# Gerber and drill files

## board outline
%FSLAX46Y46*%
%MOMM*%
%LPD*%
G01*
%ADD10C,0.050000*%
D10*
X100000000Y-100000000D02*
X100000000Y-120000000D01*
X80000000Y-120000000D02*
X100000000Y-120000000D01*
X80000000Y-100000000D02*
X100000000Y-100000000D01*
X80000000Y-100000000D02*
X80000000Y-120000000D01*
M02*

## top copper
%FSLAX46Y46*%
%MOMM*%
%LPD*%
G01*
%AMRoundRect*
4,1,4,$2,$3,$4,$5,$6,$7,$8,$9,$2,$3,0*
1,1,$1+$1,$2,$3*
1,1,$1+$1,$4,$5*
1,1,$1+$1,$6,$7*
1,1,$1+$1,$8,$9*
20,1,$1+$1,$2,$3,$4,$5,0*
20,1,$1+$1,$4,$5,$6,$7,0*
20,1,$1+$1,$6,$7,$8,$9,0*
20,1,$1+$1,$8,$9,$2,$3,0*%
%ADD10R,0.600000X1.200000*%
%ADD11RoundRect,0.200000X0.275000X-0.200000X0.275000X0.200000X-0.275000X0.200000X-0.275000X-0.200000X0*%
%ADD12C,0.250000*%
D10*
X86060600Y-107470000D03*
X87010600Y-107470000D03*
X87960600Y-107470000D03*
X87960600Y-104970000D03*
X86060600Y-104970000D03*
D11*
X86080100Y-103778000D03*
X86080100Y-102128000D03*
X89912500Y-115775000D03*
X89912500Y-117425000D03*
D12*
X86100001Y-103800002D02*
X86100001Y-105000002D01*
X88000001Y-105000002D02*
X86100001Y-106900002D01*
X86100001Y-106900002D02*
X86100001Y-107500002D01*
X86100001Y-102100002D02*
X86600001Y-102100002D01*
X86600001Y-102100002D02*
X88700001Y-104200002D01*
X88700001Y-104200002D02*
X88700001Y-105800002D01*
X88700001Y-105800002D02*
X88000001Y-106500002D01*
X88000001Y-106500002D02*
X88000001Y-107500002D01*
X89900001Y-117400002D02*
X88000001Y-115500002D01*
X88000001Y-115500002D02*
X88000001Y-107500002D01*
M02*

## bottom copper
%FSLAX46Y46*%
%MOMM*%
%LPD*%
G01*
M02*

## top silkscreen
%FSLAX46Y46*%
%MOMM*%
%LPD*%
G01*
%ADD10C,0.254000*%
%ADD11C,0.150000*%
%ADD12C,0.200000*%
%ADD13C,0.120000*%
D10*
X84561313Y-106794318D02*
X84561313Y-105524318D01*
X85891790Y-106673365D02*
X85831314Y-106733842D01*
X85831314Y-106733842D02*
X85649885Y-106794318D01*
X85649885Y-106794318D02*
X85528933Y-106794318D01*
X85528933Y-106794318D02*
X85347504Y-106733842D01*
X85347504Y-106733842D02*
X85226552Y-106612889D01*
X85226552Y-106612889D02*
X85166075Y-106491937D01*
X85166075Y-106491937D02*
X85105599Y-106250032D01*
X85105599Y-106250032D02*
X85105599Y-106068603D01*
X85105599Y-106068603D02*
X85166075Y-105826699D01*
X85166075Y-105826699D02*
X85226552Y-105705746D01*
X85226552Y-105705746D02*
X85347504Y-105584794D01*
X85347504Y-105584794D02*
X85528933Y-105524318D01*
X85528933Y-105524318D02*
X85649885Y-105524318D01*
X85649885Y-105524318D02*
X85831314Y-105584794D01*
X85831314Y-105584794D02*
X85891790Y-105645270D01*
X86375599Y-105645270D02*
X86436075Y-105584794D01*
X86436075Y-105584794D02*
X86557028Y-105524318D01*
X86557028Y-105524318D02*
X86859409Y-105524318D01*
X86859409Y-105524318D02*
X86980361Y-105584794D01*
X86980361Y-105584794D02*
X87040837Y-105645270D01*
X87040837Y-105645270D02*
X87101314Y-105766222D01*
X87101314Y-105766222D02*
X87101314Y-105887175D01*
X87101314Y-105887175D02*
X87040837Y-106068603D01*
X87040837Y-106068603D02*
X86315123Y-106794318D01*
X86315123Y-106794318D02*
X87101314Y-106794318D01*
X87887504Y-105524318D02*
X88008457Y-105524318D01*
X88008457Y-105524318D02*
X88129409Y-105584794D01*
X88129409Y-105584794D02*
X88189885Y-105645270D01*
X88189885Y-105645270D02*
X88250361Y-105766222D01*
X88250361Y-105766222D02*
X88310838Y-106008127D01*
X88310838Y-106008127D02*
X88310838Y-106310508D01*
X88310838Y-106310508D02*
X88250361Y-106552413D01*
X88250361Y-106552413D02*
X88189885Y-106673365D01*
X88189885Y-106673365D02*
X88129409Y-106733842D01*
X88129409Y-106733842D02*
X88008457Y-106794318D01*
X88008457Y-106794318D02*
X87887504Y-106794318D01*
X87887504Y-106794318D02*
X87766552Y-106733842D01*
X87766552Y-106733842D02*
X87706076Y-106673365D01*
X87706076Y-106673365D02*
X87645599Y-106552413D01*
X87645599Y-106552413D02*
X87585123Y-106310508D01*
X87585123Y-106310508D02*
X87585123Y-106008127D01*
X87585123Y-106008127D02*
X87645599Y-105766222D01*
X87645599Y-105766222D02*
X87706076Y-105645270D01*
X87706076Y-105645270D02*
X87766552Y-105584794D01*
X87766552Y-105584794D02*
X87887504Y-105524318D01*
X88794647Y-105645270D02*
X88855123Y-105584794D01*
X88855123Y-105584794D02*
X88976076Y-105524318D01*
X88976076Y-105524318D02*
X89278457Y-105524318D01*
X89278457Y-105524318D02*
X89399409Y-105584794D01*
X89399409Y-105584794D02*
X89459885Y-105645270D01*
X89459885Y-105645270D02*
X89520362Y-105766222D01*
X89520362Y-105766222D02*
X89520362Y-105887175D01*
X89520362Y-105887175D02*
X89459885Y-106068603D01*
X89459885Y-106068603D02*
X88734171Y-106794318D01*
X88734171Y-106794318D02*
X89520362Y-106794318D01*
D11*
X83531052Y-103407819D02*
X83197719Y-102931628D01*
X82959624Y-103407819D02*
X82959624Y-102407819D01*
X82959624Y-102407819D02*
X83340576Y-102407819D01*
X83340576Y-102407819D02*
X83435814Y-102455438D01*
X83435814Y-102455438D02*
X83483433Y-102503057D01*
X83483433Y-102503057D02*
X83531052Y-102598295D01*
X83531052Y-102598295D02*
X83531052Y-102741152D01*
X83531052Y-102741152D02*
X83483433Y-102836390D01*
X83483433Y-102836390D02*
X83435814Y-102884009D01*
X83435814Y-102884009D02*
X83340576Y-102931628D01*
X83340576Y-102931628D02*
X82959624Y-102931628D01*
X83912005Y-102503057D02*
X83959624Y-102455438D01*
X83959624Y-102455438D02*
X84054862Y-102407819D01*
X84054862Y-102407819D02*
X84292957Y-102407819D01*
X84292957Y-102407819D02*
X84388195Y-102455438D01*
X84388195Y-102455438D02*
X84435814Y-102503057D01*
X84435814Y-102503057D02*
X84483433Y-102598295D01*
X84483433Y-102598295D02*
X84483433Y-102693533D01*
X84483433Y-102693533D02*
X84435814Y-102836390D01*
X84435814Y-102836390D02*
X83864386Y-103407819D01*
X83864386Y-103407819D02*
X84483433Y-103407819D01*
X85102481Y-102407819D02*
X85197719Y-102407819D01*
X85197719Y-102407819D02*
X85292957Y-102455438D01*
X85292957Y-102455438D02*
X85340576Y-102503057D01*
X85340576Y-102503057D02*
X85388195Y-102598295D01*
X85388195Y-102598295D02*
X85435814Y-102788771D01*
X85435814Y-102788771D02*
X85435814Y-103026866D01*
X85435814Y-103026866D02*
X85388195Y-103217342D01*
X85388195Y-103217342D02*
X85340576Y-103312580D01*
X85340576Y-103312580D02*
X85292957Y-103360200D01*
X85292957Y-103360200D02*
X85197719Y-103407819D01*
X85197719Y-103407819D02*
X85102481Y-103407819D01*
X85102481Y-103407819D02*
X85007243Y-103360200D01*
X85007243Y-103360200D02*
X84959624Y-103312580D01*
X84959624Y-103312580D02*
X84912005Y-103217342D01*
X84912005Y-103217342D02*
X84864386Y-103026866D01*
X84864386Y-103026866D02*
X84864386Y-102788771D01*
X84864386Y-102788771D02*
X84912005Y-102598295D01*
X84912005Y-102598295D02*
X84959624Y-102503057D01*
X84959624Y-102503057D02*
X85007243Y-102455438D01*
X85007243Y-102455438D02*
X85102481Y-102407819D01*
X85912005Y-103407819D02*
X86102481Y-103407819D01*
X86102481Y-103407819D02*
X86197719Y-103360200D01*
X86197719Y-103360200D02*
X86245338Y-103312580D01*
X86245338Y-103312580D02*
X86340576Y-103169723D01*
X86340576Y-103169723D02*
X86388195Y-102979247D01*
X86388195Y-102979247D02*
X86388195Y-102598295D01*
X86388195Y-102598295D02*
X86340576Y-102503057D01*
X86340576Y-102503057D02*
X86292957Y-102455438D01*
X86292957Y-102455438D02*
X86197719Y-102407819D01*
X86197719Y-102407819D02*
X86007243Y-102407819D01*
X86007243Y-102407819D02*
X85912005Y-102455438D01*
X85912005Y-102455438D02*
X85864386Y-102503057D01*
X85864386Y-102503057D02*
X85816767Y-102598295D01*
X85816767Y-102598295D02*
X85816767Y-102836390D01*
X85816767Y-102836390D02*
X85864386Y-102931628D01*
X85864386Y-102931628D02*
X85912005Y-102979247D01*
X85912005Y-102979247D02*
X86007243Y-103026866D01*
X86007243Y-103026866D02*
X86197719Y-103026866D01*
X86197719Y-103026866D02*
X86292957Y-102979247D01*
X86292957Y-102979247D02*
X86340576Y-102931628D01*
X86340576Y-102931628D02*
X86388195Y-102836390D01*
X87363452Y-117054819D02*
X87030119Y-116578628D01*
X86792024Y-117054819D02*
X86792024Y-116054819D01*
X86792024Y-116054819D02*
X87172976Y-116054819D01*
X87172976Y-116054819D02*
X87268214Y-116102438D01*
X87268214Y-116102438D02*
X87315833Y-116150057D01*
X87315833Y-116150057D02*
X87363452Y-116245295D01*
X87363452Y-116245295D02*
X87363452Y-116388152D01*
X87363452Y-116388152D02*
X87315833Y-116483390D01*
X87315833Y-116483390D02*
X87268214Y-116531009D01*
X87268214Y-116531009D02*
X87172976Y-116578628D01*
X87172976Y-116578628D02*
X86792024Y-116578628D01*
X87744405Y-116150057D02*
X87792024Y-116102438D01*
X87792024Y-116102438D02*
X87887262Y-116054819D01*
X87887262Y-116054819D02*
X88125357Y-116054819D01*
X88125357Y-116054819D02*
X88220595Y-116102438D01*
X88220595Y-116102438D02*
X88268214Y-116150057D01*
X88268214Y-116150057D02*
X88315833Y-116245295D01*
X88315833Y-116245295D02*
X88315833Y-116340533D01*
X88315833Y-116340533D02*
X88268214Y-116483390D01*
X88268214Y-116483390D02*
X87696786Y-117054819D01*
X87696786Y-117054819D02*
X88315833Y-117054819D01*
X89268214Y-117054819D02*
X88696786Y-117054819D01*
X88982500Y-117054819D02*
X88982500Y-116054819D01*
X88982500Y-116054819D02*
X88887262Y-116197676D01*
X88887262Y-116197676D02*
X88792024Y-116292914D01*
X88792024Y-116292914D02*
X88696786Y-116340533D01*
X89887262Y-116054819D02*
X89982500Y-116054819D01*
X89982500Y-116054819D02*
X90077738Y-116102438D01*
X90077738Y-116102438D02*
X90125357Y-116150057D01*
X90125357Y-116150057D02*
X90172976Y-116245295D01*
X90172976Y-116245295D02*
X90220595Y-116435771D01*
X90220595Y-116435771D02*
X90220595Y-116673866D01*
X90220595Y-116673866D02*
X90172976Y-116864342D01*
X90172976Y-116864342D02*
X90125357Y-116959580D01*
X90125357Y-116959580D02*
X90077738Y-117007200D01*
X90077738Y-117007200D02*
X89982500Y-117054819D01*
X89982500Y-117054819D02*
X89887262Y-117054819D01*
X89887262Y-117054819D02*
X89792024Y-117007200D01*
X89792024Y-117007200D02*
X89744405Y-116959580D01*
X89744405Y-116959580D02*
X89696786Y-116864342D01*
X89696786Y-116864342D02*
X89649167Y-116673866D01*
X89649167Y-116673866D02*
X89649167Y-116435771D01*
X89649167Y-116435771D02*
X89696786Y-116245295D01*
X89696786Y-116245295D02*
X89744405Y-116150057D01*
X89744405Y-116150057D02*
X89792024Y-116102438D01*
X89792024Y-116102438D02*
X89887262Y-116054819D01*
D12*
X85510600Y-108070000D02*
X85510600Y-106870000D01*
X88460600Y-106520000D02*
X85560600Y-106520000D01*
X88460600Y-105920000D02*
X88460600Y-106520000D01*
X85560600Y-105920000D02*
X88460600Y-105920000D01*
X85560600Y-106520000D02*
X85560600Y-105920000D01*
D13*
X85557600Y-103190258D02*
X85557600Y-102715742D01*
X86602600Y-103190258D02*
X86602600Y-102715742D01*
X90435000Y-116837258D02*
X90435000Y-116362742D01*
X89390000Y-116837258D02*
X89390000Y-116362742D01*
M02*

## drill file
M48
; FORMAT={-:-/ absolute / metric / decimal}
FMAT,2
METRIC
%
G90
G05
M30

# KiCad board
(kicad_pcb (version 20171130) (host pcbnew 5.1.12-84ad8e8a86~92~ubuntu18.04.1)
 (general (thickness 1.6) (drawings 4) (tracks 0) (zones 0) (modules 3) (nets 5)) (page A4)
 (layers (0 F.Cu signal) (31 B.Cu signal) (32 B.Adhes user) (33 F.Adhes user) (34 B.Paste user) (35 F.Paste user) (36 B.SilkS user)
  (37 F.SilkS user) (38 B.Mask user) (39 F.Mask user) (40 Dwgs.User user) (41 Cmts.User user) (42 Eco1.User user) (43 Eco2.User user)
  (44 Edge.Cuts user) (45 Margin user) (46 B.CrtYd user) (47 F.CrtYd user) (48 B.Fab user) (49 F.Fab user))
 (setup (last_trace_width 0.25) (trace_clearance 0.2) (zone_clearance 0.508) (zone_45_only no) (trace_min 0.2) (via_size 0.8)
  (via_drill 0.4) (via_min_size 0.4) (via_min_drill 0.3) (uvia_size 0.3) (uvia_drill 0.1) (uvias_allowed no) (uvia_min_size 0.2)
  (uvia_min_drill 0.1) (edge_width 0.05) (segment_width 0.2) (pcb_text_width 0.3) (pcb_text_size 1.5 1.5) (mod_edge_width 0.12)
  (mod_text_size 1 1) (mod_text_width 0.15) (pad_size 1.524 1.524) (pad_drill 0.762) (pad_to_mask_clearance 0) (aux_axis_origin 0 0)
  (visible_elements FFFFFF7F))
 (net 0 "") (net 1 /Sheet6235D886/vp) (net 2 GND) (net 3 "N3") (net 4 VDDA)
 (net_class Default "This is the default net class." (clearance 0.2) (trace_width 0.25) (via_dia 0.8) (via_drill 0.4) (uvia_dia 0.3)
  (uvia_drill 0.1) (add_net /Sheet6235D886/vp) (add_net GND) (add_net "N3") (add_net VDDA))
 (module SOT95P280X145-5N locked (layer F.Cu) (at 87.010600 106.220000 90.000000)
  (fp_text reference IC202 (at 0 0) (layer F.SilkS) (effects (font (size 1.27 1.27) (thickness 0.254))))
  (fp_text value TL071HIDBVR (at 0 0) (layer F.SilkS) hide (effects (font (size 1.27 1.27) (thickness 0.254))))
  (fp_line (start -1.85 -1.5) (end -0.65 -1.5) (layer F.SilkS) (width 0.2))
  (fp_line (start -0.3 1.45) (end -0.3 -1.45) (layer F.SilkS) (width 0.2))
  (fp_line (start 0.3 1.45) (end -0.3 1.45) (layer F.SilkS) (width 0.2))
  (fp_line (start 0.3 -1.45) (end 0.3 1.45) (layer F.SilkS) (width 0.2))
  (fp_line (start -0.3 -1.45) (end 0.3 -1.45) (layer F.SilkS) (width 0.2))
  (pad 1 smd rect (at -1.25 -0.95 180.000000) (size 0.6 1.2) (layers F.Cu F.Mask F.Paste) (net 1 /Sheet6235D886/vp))
  (pad 2 smd rect (at -1.25 0 180.000000) (size 0.6 1.2) (layers F.Cu F.Mask F.Paste) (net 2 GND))
  (pad 3 smd rect (at -1.25 0.95 180.000000) (size 0.6 1.2) (layers F.Cu F.Mask F.Paste) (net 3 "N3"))
  (pad 4 smd rect (at 1.25 0.95 180.000000) (size 0.6 1.2) (layers F.Cu F.Mask F.Paste) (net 1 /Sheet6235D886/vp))
  (pad 5 smd rect (at 1.25 -0.95 180.000000) (size 0.6 1.2) (layers F.Cu F.Mask F.Paste) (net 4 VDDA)))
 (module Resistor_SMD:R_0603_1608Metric (layer F.Cu) (at 86.080100 102.953000 90.000000)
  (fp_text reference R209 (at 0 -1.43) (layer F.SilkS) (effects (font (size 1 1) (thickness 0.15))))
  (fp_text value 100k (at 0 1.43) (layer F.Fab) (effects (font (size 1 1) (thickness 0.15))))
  (fp_line (start -0.237258 -0.5225) (end 0.237258 -0.5225) (layer F.SilkS) (width 0.12))
  (fp_line (start -0.237258 0.5225) (end 0.237258 0.5225) (layer F.SilkS) (width 0.12))
  (pad 1 smd roundrect (at -0.825 0 90.000000) (size 0.8 0.95) (layers F.Cu F.Mask F.Paste) (roundrect_rratio 0.25) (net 4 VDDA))
  (pad 2 smd roundrect (at 0.825 0 90.000000) (size 0.8 0.95) (layers F.Cu F.Mask F.Paste) (roundrect_rratio 0.25) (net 3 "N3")))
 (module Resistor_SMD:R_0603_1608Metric (layer F.Cu) (at 89.912500 116.600000 90.000000)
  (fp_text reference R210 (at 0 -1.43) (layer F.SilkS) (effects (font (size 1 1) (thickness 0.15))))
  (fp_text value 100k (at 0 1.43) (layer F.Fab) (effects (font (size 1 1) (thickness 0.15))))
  (fp_line (start -0.237258 0.5225) (end 0.237258 0.5225) (layer F.SilkS) (width 0.12))
  (fp_line (start -0.237258 -0.5225) (end 0.237258 -0.5225) (layer F.SilkS) (width 0.12))
  (pad 2 smd roundrect (at 0.825 0 90.000000) (size 0.8 0.95) (layers F.Cu F.Mask F.Paste) (roundrect_rratio 0.25) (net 2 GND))
  (pad 1 smd roundrect (at -0.825 0 90.000000) (size 0.8 0.95) (layers F.Cu F.Mask F.Paste) (roundrect_rratio 0.25) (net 3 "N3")))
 (gr_line (start 100 100) (end 100 120) (layer Edge.Cuts) (width 0.05))
 (gr_line (start 80 120) (end 100 120) (layer Edge.Cuts) (width 0.05))
 (gr_line (start 80 100) (end 100 100) (layer Edge.Cuts) (width 0.05))
 (gr_line (start 80 100) (end 80 120) (layer Edge.Cuts) (width 0.05))
 (segment (start 86.100001 103.800002) (end 86.100001 105.000002) (width 0.250000) (layer F.Cu) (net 4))
 (segment (start 88.000001 105.000002) (end 86.100001 106.900002) (width 0.250000) (layer F.Cu) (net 1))
 (segment (start 86.100001 106.900002) (end 86.100001 107.500002) (width 0.250000) (layer F.Cu) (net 1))
 (segment (start 86.100001 102.100002) (end 86.600001 102.100002) (width 0.250000) (layer F.Cu) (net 3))
 (segment (start 86.600001 102.100002) (end 88.700001 104.200002) (width 0.250000) (layer F.Cu) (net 3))
 (segment (start 88.700001 104.200002) (end 88.700001 105.800002) (width 0.250000) (layer F.Cu) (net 3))
 (segment (start 88.700001 105.800002) (end 88.000001 106.500002) (width 0.250000) (layer F.Cu) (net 3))
 (segment (start 88.000001 106.500002) (end 88.000001 107.500002) (width 0.250000) (layer F.Cu) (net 3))
 (segment (start 89.900001 117.400002) (end 88.000001 115.500002) (width 0.250000) (layer F.Cu) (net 3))
 (segment (start 88.000001 115.500002) (end 88.000001 107.500002) (width 0.250000) (layer F.Cu) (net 3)))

